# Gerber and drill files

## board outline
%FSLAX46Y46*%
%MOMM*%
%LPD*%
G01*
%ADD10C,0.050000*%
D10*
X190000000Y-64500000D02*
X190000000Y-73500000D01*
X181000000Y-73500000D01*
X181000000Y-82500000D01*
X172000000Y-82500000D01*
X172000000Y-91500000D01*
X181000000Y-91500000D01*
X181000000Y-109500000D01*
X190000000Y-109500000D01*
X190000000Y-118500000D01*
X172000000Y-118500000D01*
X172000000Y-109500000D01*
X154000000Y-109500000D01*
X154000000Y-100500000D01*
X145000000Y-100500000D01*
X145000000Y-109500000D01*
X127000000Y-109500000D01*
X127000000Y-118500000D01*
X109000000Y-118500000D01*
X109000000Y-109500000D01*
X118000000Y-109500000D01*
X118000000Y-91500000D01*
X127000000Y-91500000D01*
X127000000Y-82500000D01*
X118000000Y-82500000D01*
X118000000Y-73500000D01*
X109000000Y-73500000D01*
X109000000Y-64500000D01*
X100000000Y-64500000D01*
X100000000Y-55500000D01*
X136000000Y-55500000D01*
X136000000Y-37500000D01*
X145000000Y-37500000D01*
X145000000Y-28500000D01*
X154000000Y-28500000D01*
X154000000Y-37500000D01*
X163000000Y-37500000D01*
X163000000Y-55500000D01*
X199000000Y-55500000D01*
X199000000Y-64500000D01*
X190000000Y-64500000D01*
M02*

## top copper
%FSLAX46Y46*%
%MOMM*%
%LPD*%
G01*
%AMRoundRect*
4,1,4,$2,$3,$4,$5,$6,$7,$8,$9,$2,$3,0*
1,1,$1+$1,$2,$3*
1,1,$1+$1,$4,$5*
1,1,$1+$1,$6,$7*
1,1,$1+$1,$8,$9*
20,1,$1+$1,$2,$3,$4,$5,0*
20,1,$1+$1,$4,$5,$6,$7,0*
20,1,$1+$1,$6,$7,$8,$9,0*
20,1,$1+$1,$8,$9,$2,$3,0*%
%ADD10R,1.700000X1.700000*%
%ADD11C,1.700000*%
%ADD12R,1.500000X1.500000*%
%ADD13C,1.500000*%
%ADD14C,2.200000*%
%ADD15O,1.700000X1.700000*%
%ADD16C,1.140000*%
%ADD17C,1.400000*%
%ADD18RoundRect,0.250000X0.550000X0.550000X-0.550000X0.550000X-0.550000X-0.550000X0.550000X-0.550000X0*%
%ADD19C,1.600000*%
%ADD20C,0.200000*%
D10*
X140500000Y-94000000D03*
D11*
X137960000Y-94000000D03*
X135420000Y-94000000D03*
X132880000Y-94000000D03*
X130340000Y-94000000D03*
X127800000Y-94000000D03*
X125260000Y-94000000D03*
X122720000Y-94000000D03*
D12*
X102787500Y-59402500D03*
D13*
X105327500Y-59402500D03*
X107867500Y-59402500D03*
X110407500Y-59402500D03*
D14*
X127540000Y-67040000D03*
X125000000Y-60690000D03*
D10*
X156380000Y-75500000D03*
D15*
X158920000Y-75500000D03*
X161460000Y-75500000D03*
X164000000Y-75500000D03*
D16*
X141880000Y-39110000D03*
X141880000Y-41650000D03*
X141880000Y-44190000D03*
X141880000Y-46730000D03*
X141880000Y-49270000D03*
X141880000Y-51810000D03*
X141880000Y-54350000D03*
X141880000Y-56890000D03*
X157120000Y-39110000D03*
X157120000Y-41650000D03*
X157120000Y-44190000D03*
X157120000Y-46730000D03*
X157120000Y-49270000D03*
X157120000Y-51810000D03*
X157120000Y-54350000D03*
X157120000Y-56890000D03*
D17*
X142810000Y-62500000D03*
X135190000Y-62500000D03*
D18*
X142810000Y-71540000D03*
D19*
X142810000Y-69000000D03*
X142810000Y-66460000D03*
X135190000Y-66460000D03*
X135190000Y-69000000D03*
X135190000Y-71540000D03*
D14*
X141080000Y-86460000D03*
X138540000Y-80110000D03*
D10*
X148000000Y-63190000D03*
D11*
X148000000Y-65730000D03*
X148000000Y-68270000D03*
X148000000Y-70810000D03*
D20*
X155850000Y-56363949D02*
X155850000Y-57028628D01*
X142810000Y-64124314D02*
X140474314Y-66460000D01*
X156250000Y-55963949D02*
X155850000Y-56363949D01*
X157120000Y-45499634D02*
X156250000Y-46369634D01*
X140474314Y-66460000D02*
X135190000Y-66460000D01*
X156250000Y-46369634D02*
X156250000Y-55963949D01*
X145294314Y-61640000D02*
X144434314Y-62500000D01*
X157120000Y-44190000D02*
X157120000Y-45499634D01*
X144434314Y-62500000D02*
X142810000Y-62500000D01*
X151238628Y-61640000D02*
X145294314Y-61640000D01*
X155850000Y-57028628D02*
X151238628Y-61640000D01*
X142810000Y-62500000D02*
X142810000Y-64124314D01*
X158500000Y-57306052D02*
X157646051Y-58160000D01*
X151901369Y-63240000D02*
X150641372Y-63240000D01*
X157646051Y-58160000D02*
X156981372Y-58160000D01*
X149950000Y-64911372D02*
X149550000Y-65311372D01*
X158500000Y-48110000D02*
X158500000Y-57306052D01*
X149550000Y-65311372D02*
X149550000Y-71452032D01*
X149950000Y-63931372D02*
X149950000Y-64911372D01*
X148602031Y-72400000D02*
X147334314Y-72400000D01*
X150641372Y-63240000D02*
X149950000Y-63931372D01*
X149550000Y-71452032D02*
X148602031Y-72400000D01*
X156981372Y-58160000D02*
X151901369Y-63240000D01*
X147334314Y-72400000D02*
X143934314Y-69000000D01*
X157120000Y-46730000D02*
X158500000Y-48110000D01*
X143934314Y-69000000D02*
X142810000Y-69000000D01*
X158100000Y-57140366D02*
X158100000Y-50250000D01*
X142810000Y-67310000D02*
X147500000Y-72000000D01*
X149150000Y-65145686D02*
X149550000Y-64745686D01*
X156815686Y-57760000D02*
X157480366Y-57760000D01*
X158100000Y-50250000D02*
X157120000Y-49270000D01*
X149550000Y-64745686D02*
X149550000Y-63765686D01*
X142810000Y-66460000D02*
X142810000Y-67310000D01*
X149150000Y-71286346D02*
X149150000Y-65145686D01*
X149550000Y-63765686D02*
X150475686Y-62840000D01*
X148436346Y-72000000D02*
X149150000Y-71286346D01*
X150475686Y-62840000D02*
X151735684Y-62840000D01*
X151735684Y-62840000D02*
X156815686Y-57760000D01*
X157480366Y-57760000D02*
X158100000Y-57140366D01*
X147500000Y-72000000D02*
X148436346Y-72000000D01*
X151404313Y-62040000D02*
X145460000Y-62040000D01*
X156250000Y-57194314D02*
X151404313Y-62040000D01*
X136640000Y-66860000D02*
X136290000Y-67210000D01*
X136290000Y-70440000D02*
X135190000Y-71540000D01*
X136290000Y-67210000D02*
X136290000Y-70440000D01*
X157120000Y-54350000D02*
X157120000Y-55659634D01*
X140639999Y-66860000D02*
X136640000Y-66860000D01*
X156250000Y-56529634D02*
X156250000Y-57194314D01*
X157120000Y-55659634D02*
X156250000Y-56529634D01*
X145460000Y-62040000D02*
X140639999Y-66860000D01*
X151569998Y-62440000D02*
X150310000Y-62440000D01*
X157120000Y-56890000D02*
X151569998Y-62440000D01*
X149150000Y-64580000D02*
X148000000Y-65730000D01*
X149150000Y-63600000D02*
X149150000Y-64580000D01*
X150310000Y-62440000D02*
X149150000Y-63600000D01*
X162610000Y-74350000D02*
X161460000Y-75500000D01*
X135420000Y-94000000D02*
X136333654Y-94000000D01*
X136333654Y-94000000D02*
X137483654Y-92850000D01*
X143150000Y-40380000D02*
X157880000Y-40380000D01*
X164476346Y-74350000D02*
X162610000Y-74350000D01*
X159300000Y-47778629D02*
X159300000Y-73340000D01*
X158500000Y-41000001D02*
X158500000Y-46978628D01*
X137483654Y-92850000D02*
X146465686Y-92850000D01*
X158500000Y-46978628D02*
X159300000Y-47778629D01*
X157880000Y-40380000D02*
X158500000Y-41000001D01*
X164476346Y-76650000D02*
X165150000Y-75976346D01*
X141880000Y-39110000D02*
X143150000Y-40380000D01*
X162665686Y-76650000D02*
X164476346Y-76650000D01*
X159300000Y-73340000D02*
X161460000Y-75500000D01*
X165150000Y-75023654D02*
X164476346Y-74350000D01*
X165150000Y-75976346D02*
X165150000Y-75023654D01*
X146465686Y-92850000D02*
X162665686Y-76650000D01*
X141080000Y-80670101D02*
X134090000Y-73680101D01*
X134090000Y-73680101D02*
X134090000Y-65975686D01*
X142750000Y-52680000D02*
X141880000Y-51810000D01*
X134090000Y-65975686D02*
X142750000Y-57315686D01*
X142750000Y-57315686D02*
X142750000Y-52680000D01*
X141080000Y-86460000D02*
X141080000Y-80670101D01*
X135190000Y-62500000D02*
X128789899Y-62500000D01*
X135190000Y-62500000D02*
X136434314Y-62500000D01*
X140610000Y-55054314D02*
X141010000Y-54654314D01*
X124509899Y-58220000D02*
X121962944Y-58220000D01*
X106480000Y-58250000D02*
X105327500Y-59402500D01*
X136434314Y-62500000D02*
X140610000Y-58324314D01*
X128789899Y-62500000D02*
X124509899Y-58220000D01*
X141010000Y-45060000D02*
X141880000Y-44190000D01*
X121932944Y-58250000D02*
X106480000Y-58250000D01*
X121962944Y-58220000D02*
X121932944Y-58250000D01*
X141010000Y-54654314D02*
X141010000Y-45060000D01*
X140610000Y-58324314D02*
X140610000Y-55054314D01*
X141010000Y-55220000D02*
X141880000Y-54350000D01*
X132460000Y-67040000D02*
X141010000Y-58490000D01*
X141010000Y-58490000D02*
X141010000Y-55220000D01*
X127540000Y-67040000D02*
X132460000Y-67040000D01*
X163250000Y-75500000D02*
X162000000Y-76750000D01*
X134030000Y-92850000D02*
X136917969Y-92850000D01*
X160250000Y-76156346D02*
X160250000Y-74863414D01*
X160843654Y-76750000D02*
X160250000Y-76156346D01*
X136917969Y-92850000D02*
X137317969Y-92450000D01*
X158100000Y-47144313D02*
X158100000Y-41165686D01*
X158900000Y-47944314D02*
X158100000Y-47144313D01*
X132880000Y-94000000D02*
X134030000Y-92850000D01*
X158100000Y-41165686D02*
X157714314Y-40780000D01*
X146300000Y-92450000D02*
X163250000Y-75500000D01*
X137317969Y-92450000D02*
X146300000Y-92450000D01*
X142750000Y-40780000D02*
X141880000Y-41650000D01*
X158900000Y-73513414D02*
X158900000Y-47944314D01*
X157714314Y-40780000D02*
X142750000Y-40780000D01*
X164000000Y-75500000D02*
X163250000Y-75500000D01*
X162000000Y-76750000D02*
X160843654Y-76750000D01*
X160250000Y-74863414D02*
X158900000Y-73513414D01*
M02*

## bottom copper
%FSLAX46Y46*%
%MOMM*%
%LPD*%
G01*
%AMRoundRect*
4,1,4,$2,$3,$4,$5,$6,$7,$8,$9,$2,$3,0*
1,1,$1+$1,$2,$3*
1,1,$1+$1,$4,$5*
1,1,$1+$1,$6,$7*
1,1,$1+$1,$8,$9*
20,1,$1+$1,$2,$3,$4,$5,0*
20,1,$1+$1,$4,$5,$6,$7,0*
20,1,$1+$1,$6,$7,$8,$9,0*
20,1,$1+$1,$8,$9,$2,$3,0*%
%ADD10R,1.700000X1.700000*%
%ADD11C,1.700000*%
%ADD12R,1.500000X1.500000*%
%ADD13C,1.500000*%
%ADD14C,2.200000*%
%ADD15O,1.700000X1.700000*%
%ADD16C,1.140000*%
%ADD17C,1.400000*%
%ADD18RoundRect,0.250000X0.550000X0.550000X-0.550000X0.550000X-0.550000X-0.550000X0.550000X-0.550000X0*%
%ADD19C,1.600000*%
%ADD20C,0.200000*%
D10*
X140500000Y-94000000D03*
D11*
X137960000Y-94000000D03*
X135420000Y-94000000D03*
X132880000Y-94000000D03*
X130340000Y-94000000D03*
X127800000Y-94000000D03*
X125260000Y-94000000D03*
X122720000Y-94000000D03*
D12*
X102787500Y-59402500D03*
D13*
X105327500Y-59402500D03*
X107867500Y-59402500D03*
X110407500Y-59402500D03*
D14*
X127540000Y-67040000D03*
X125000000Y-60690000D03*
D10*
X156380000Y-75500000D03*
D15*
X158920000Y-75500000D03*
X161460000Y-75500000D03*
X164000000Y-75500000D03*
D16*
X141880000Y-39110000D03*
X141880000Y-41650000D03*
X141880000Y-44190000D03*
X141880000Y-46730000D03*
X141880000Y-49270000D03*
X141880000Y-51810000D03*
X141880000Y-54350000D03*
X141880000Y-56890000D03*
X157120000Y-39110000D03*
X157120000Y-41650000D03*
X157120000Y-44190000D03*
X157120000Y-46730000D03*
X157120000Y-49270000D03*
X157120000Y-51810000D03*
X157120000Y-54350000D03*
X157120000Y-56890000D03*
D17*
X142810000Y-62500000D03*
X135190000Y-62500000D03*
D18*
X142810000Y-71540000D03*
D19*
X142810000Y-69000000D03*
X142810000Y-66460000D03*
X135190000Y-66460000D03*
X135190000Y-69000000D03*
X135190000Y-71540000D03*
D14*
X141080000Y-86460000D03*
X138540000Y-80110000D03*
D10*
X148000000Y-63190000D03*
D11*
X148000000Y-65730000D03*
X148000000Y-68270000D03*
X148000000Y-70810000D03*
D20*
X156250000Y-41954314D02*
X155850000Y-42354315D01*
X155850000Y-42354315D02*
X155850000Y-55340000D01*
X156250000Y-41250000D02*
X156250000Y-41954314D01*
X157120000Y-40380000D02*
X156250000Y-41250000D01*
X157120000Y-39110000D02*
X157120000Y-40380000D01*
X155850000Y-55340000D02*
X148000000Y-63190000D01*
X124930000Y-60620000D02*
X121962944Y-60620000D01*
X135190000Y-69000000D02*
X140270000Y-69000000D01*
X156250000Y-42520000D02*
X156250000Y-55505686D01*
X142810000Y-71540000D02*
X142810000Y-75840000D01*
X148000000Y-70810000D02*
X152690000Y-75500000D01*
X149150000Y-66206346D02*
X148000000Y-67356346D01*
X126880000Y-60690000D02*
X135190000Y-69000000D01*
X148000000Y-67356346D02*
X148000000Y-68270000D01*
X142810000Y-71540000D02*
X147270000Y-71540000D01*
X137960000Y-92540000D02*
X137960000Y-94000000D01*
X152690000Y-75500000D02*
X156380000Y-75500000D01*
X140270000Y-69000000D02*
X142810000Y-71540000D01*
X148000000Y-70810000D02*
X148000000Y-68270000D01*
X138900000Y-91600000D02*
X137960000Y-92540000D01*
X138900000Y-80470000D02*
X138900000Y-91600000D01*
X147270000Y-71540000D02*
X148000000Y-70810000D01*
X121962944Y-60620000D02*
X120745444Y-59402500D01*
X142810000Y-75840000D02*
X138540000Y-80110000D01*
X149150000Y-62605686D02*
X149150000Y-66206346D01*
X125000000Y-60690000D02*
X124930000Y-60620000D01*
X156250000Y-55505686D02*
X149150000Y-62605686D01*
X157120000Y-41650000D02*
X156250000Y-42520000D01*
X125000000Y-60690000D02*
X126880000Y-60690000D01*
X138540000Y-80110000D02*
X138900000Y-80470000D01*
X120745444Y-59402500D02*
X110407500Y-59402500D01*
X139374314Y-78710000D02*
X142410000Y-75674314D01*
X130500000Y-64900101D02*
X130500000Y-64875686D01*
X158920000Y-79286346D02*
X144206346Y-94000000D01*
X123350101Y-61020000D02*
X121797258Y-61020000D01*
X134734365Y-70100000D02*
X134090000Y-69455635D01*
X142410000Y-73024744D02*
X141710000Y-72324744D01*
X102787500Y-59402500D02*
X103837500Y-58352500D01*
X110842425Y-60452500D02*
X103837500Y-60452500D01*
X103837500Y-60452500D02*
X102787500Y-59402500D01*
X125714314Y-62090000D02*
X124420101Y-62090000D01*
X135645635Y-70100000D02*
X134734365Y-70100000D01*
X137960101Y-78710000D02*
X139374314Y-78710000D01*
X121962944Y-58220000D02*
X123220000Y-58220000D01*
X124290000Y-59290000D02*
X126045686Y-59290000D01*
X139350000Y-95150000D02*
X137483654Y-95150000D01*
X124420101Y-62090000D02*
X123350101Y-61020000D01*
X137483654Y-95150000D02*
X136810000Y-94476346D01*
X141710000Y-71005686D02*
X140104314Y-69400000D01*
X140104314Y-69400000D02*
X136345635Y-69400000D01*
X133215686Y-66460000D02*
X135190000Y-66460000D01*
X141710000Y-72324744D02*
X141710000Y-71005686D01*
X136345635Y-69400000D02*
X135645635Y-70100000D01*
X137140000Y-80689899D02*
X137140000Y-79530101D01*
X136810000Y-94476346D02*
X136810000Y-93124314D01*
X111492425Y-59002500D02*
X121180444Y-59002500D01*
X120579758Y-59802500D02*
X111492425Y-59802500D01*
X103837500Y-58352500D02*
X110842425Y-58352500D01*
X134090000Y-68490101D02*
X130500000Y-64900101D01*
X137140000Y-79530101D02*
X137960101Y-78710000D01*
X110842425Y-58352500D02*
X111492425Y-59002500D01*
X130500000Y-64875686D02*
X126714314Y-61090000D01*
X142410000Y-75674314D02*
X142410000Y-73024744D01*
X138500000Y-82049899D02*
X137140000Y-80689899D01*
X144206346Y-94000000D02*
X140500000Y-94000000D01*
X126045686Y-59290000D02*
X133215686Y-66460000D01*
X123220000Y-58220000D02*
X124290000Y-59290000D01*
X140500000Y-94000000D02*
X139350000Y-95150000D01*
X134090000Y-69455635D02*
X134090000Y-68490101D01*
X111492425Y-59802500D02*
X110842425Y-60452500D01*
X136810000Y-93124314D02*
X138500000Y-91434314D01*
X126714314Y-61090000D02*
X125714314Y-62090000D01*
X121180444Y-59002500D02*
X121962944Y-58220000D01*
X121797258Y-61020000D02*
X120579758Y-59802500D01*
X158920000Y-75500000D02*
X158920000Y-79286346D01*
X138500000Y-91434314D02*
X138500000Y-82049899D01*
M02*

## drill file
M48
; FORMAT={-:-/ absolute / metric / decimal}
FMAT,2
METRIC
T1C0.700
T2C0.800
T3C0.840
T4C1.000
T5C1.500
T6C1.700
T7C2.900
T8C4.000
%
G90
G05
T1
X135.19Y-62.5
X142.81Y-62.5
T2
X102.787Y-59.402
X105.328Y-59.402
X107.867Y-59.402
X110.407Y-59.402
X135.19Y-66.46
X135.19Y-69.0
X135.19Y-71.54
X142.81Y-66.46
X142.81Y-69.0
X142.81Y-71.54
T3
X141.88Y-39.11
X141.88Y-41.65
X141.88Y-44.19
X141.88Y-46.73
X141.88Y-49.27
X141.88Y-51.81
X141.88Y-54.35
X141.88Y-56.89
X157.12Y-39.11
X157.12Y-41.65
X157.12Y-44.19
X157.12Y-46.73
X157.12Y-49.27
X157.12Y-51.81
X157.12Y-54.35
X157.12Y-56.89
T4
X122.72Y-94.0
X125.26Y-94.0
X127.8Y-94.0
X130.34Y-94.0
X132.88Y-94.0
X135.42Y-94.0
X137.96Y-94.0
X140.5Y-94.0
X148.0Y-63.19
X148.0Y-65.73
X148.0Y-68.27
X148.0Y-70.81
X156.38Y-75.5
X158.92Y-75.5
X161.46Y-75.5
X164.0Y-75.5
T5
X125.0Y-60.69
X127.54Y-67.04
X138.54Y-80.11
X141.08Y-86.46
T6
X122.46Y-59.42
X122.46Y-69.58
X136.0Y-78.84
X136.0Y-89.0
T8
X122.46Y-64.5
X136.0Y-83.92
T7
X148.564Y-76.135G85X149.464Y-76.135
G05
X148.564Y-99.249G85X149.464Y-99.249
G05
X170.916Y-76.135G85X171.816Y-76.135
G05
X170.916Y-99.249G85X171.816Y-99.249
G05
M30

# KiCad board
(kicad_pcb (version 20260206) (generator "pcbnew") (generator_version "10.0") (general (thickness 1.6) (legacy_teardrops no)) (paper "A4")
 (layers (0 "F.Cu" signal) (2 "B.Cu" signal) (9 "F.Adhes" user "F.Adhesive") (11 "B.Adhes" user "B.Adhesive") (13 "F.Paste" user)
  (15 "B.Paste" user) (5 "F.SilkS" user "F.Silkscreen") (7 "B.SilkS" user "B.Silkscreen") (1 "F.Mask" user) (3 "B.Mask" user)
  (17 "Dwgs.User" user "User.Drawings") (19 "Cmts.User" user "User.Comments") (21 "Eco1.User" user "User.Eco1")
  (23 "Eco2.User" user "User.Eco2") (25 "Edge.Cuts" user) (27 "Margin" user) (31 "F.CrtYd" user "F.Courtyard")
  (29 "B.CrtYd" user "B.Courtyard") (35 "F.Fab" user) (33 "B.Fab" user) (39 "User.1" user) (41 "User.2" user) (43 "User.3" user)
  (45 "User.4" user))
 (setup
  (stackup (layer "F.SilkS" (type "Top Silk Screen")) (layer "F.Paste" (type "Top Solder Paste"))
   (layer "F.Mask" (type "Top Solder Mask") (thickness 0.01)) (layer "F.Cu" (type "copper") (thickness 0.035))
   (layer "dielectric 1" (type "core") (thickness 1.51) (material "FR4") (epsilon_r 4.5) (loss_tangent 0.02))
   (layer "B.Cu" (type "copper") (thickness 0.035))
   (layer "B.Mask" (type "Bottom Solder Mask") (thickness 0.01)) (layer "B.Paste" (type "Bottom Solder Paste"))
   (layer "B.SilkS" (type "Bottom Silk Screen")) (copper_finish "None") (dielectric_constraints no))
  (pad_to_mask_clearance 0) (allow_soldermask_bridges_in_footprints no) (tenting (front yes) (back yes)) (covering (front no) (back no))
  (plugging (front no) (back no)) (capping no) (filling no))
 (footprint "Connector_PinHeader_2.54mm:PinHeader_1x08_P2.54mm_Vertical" (layer "F.Cu") (at 140.5 94 -90)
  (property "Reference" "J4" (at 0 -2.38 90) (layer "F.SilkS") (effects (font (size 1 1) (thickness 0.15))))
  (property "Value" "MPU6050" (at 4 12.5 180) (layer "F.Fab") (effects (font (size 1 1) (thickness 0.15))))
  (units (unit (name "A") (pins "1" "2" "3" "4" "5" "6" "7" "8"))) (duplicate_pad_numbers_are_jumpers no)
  (pad "1" thru_hole rect (at 0 0 270) (size 1.7 1.7) (drill 1) (layers "*.Cu" "*.Mask") (remove_unused_layers no) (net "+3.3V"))
  (pad "2" thru_hole circle (at 0 2.54 270) (size 1.7 1.7) (drill 1) (layers "*.Cu" "*.Mask") (remove_unused_layers no) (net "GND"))
  (pad "3" thru_hole circle (at 0 5.08 270) (size 1.7 1.7) (drill 1) (layers "*.Cu" "*.Mask") (remove_unused_layers no) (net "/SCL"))
  (pad "4" thru_hole circle (at 0 7.62 270) (size 1.7 1.7) (drill 1) (layers "*.Cu" "*.Mask") (remove_unused_layers no) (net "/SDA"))
  (pad "5" thru_hole circle (at 0 10.16 270) (size 1.7 1.7) (drill 1) (layers "*.Cu" "*.Mask") (remove_unused_layers no)
   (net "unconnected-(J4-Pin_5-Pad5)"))
  (pad "6" thru_hole circle (at 0 12.7 270) (size 1.7 1.7) (drill 1) (layers "*.Cu" "*.Mask") (remove_unused_layers no)
   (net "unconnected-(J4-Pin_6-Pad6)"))
  (pad "7" thru_hole circle (at 0 15.24 270) (size 1.7 1.7) (drill 1) (layers "*.Cu" "*.Mask") (remove_unused_layers no)
   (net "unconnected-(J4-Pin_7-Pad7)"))
  (pad "8" thru_hole circle (at 0 17.78 270) (size 1.7 1.7) (drill 1) (layers "*.Cu" "*.Mask") (remove_unused_layers no)
   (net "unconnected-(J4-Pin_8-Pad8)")))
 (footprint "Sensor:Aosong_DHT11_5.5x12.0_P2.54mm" (layer "F.Cu") (at 102.7875 59.4025 90)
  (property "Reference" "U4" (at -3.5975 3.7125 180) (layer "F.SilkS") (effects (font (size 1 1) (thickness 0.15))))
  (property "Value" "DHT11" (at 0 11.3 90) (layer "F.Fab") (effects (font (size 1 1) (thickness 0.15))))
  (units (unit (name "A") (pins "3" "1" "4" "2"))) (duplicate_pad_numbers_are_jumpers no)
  (pad "1" thru_hole rect (at 0 0 90) (size 1.5 1.5) (drill 0.8) (layers "*.Cu" "*.Mask") (remove_unused_layers no) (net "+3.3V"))
  (pad "2" thru_hole circle (at 0 2.54 90) (size 1.5 1.5) (drill 0.8) (layers "*.Cu" "*.Mask") (remove_unused_layers no) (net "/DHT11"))
  (pad "3" thru_hole circle (at 0 5.08 90) (size 1.5 1.5) (drill 0.8) (layers "*.Cu" "*.Mask") (remove_unused_layers no)
   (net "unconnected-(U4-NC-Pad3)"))
  (pad "4" thru_hole circle (at 0 7.62 90) (size 1.5 1.5) (drill 0.8) (layers "*.Cu" "*.Mask") (remove_unused_layers no) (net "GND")))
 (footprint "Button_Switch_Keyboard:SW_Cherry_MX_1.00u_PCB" (layer "F.Cu") (at 127.54 67.04 -90)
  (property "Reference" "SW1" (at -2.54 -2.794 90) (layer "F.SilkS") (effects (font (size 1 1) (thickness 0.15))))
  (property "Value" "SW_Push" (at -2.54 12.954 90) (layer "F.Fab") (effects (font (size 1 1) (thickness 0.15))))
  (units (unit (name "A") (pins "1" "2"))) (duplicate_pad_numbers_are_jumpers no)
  (pad "" np_thru_hole circle (at -7.62 5.08 270) (size 1.7 1.7) (drill 1.7) (layers "*.Cu" "*.Mask"))
  (pad "" np_thru_hole circle (at -2.54 5.08 270) (size 4 4) (drill 4) (layers "*.Cu" "*.Mask"))
  (pad "" np_thru_hole circle (at 2.54 5.08 270) (size 1.7 1.7) (drill 1.7) (layers "*.Cu" "*.Mask"))
  (pad "1" thru_hole circle (at 0 0 270) (size 2.2 2.2) (drill 1.5) (layers "*.Cu" "*.Mask") (remove_unused_layers no) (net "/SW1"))
  (pad "2" thru_hole circle (at -6.35 2.54 270) (size 2.2 2.2) (drill 1.5) (layers "*.Cu" "*.Mask") (remove_unused_layers no) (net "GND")))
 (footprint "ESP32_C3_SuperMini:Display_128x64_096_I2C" (layer "F.Cu") (at 160.19 75.5)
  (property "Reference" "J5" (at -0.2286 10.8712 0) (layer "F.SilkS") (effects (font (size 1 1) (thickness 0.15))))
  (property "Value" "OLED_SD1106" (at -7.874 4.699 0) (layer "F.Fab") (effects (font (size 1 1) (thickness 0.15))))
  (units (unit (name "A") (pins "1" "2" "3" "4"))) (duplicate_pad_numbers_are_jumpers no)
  (pad "" np_thru_hole oval (at -11.176 0.635) (size 3.8 2.9) (drill oval 3.8 2.9) (layers "*.Cu" "*.Mask"))
  (pad "" np_thru_hole oval (at -11.176 23.749) (size 3.8 2.9) (drill oval 3.8 2.9) (layers "*.Cu" "*.Mask"))
  (pad "" np_thru_hole oval (at 11.176 0.635) (size 3.8 2.9) (drill oval 3.8 2.9) (layers "*.Cu" "*.Mask"))
  (pad "" np_thru_hole oval (at 11.176 23.749) (size 3.8 2.9) (drill oval 3.8 2.9) (layers "*.Cu" "*.Mask"))
  (pad "1" thru_hole rect (at -3.81 0 90) (size 1.7 1.7) (drill 1) (layers "*.Cu" "*.Mask") (remove_unused_layers no) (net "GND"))
  (pad "2" thru_hole oval (at -1.27 0 90) (size 1.7 1.7) (drill 1) (layers "*.Cu" "*.Mask") (remove_unused_layers no) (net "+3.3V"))
  (pad "3" thru_hole oval (at 1.27 0 90) (size 1.7 1.7) (drill 1) (layers "*.Cu" "*.Mask") (remove_unused_layers no) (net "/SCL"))
  (pad "4" thru_hole oval (at 3.81 0 90) (size 1.7 1.7) (drill 1) (layers "*.Cu" "*.Mask") (remove_unused_layers no) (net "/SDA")))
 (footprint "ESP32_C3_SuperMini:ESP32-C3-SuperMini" (layer "F.Cu") (at 149.5 48)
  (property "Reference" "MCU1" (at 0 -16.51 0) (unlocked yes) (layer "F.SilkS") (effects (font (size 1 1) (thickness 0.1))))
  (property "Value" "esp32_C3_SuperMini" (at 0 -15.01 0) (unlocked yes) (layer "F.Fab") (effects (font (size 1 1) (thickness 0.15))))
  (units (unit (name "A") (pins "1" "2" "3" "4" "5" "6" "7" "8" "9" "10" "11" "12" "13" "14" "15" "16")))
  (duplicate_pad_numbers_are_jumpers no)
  (pad "1" thru_hole circle (at -7.62 -8.89) (size 1.14 1.14) (drill 0.84) (layers "*.Cu" "*.Mask") (remove_unused_layers no) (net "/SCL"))
  (pad "2" thru_hole circle (at -7.62 -6.35) (size 1.14 1.14) (drill 0.84) (layers "*.Cu" "*.Mask") (remove_unused_layers no) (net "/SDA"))
  (pad "3" thru_hole circle (at -7.62 -3.81) (size 1.14 1.14) (drill 0.84) (layers "*.Cu" "*.Mask") (remove_unused_layers no) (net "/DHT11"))
  (pad "4" thru_hole circle (at -7.62 -1.27) (size 1.14 1.14) (drill 0.84) (layers "*.Cu" "*.Mask") (remove_unused_layers no)
   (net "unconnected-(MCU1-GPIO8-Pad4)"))
  (pad "5" thru_hole circle (at -7.62 1.27) (size 1.14 1.14) (drill 0.84) (layers "*.Cu" "*.Mask") (remove_unused_layers no)
   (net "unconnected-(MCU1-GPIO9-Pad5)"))
  (pad "6" thru_hole circle (at -7.62 3.81) (size 1.14 1.14) (drill 0.84) (layers "*.Cu" "*.Mask") (remove_unused_layers no) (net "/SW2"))
  (pad "7" thru_hole circle (at -7.62 6.35) (size 1.14 1.14) (drill 0.84) (layers "*.Cu" "*.Mask") (remove_unused_layers no) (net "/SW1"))
  (pad "8" thru_hole circle (at -7.62 8.89) (size 1.14 1.14) (drill 0.84) (layers "*.Cu" "*.Mask") (remove_unused_layers no)
   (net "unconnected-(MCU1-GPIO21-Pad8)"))
  (pad "9" thru_hole circle (at 7.62 -8.89) (size 1.14 1.14) (drill 0.84) (layers "*.Cu" "*.Mask") (remove_unused_layers no) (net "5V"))
  (pad "10" thru_hole circle (at 7.62 -6.35) (size 1.14 1.14) (drill 0.84) (layers "*.Cu" "*.Mask") (remove_unused_layers no) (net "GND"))
  (pad "11" thru_hole circle (at 7.62 -3.81) (size 1.14 1.14) (drill 0.84) (layers "*.Cu" "*.Mask") (remove_unused_layers no) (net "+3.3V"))
  (pad "12" thru_hole circle (at 7.62 -1.27) (size 1.14 1.14) (drill 0.84) (layers "*.Cu" "*.Mask") (remove_unused_layers no) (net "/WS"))
  (pad "13" thru_hole circle (at 7.62 1.27) (size 1.14 1.14) (drill 0.84) (layers "*.Cu" "*.Mask") (remove_unused_layers no) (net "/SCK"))
  (pad "14" thru_hole circle (at 7.62 3.81) (size 1.14 1.14) (drill 0.84) (layers "*.Cu" "*.Mask") (remove_unused_layers no)
   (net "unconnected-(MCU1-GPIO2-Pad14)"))
  (pad "15" thru_hole circle (at 7.62 6.35) (size 1.14 1.14) (drill 0.84) (layers "*.Cu" "*.Mask") (remove_unused_layers no) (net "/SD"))
  (pad "16" thru_hole circle (at 7.62 8.89) (size 1.14 1.14) (drill 0.84) (layers "*.Cu" "*.Mask") (remove_unused_layers no) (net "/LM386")))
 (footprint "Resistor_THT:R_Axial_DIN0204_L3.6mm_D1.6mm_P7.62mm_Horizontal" (layer "F.Cu") (at 142.81 62.5 180)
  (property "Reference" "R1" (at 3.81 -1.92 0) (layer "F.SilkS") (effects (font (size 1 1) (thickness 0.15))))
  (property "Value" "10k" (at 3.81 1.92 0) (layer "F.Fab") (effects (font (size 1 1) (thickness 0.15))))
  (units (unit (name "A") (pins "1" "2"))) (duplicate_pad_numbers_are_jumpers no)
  (pad "1" thru_hole circle (at 0 0 180) (size 1.4 1.4) (drill 0.7) (layers "*.Cu" "*.Mask") (remove_unused_layers no) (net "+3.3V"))
  (pad "2" thru_hole circle (at 7.62 0 180) (size 1.4 1.4) (drill 0.7) (layers "*.Cu" "*.Mask") (remove_unused_layers no) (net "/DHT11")))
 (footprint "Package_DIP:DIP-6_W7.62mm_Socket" (layer "F.Cu") (at 142.81 71.54 180)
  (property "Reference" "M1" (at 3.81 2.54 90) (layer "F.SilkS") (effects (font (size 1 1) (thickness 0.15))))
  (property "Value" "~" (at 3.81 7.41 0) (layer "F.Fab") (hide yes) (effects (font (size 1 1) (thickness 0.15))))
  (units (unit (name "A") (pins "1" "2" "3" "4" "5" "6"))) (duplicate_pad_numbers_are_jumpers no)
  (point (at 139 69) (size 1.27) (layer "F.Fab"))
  (pad "1" thru_hole roundrect (at 0 0 180) (size 1.6 1.6) (drill 0.8) (layers "*.Cu" "*.Mask") (remove_unused_layers no)
   (roundrect_rratio 0.15625) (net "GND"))
  (pad "2" thru_hole circle (at 0 2.54 180) (size 1.6 1.6) (drill 0.8) (layers "*.Cu" "*.Mask") (remove_unused_layers no) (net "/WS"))
  (pad "3" thru_hole circle (at 0 5.08 180) (size 1.6 1.6) (drill 0.8) (layers "*.Cu" "*.Mask") (remove_unused_layers no) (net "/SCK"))
  (pad "4" thru_hole circle (at 7.62 5.08 180) (size 1.6 1.6) (drill 0.8) (layers "*.Cu" "*.Mask") (remove_unused_layers no) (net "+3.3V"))
  (pad "5" thru_hole circle (at 7.62 2.54 180) (size 1.6 1.6) (drill 0.8) (layers "*.Cu" "*.Mask") (remove_unused_layers no) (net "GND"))
  (pad "6" thru_hole circle (at 7.62 0 180) (size 1.6 1.6) (drill 0.8) (layers "*.Cu" "*.Mask") (remove_unused_layers no) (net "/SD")))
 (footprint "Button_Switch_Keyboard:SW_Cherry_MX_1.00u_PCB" (layer "F.Cu") (at 141.08 86.46 -90)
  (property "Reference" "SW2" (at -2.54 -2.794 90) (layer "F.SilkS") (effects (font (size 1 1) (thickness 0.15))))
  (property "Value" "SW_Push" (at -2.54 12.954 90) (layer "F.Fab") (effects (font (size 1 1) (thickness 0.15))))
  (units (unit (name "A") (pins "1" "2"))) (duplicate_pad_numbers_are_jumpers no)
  (pad "" np_thru_hole circle (at -7.62 5.08 270) (size 1.7 1.7) (drill 1.7) (layers "*.Cu" "*.Mask"))
  (pad "" np_thru_hole circle (at -2.54 5.08 270) (size 4 4) (drill 4) (layers "*.Cu" "*.Mask"))
  (pad "" np_thru_hole circle (at 2.54 5.08 270) (size 1.7 1.7) (drill 1.7) (layers "*.Cu" "*.Mask"))
  (pad "1" thru_hole circle (at 0 0 270) (size 2.2 2.2) (drill 1.5) (layers "*.Cu" "*.Mask") (remove_unused_layers no) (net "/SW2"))
  (pad "2" thru_hole circle (at -6.35 2.54 270) (size 2.2 2.2) (drill 1.5) (layers "*.Cu" "*.Mask") (remove_unused_layers no) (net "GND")))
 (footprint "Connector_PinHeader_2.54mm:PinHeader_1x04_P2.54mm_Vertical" (layer "F.Cu") (at 148 63.19)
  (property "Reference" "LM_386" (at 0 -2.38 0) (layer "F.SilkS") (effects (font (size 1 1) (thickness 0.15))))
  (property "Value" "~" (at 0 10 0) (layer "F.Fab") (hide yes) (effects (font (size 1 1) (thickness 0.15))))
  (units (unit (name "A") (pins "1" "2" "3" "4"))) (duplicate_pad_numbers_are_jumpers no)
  (pad "1" thru_hole rect (at 0 0) (size 1.7 1.7) (drill 1) (layers "*.Cu" "*.Mask") (remove_unused_layers no) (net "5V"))
  (pad "2" thru_hole circle (at 0 2.54) (size 1.7 1.7) (drill 1) (layers "*.Cu" "*.Mask") (remove_unused_layers no) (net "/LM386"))
  (pad "3" thru_hole circle (at 0 5.08) (size 1.7 1.7) (drill 1) (layers "*.Cu" "*.Mask") (remove_unused_layers no) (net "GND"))
  (pad "4" thru_hole circle (at 0 7.62) (size 1.7 1.7) (drill 1) (layers "*.Cu" "*.Mask") (remove_unused_layers no) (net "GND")))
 (gr_poly
  (pts (xy 190 64.5) (xy 190 73.5) (xy 181 73.5) (xy 181 82.5) (xy 172 82.5) (xy 172 91.5) (xy 181 91.5) (xy 181 109.5) (xy 190 109.5)
   (xy 190 118.5) (xy 172 118.5) (xy 172 109.5) (xy 154 109.5) (xy 154 100.5) (xy 145 100.5) (xy 145 109.5) (xy 127 109.5) (xy 127 118.5)
   (xy 109 118.5) (xy 109 109.5) (xy 118 109.5) (xy 118 91.5) (xy 127 91.5) (xy 127 82.5) (xy 118 82.5) (xy 118 73.5) (xy 109 73.5)
   (xy 109 64.5) (xy 100 64.5) (xy 100 55.5) (xy 136 55.5) (xy 136 37.5) (xy 145 37.5) (xy 145 28.5) (xy 154 28.5) (xy 154 37.5)
   (xy 163 37.5) (xy 163 55.5) (xy 199 55.5) (xy 199 64.5))
  (stroke (width 0.05) (type solid)) (fill no) (layer "Edge.Cuts"))
 (segment (start 156.25 41.954314) (end 155.85 42.354315) (width 0.2) (layer "B.Cu") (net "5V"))
 (segment (start 155.85 42.354315) (end 155.85 55.34) (width 0.2) (layer "B.Cu") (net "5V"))
 (segment (start 156.25 41.25) (end 156.25 41.954314) (width 0.2) (layer "B.Cu") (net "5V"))
 (segment (start 157.12 40.38) (end 156.25 41.25) (width 0.2) (layer "B.Cu") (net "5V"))
 (segment (start 157.12 39.11) (end 157.12 40.38) (width 0.2) (layer "B.Cu") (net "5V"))
 (segment (start 155.85 55.34) (end 148 63.19) (width 0.2) (layer "B.Cu") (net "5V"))
 (segment (start 124.93 60.62) (end 121.962944 60.62) (width 0.2) (layer "B.Cu") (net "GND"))
 (segment (start 135.19 69) (end 140.27 69) (width 0.2) (layer "B.Cu") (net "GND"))
 (segment (start 156.25 42.52) (end 156.25 55.505686) (width 0.2) (layer "B.Cu") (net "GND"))
 (segment (start 142.81 71.54) (end 142.81 75.84) (width 0.2) (layer "B.Cu") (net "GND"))
 (segment (start 148 70.81) (end 152.69 75.5) (width 0.2) (layer "B.Cu") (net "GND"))
 (segment (start 149.15 66.206346) (end 148 67.356346) (width 0.2) (layer "B.Cu") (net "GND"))
 (segment (start 126.88 60.69) (end 135.19 69) (width 0.2) (layer "B.Cu") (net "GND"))
 (segment (start 148 67.356346) (end 148 68.27) (width 0.2) (layer "B.Cu") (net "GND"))
 (segment (start 142.81 71.54) (end 147.27 71.54) (width 0.2) (layer "B.Cu") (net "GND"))
 (segment (start 137.96 92.54) (end 137.96 94) (width 0.2) (layer "B.Cu") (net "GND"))
 (segment (start 152.69 75.5) (end 156.38 75.5) (width 0.2) (layer "B.Cu") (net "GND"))
 (segment (start 140.27 69) (end 142.81 71.54) (width 0.2) (layer "B.Cu") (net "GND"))
 (segment (start 148 70.81) (end 148 68.27) (width 0.2) (layer "B.Cu") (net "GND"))
 (segment (start 138.9 91.6) (end 137.96 92.54) (width 0.2) (layer "B.Cu") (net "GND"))
 (segment (start 138.9 80.47) (end 138.9 91.6) (width 0.2) (layer "B.Cu") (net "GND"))
 (segment (start 147.27 71.54) (end 148 70.81) (width 0.2) (layer "B.Cu") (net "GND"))
 (segment (start 121.962944 60.62) (end 120.745444 59.4025) (width 0.2) (layer "B.Cu") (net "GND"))
 (segment (start 142.81 75.84) (end 138.54 80.11) (width 0.2) (layer "B.Cu") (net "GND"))
 (segment (start 149.15 62.605686) (end 149.15 66.206346) (width 0.2) (layer "B.Cu") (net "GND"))
 (segment (start 125 60.69) (end 124.93 60.62) (width 0.2) (layer "B.Cu") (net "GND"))
 (segment (start 156.25 55.505686) (end 149.15 62.605686) (width 0.2) (layer "B.Cu") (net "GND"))
 (segment (start 157.12 41.65) (end 156.25 42.52) (width 0.2) (layer "B.Cu") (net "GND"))
 (segment (start 125 60.69) (end 126.88 60.69) (width 0.2) (layer "B.Cu") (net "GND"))
 (segment (start 138.54 80.11) (end 138.9 80.47) (width 0.2) (layer "B.Cu") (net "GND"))
 (segment (start 120.745444 59.4025) (end 110.4075 59.4025) (width 0.2) (layer "B.Cu") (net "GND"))
 (segment (start 155.85 56.363949) (end 155.85 57.028628) (width 0.2) (layer "F.Cu") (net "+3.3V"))
 (segment (start 142.81 64.124314) (end 140.474314 66.46) (width 0.2) (layer "F.Cu") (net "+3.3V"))
 (segment (start 156.25 55.963949) (end 155.85 56.363949) (width 0.2) (layer "F.Cu") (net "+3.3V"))
 (segment (start 157.12 45.499634) (end 156.25 46.369634) (width 0.2) (layer "F.Cu") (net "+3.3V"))
 (segment (start 140.474314 66.46) (end 135.19 66.46) (width 0.2) (layer "F.Cu") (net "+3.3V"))
 (segment (start 156.25 46.369634) (end 156.25 55.963949) (width 0.2) (layer "F.Cu") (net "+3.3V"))
 (segment (start 145.294314 61.64) (end 144.434314 62.5) (width 0.2) (layer "F.Cu") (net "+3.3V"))
 (segment (start 157.12 44.19) (end 157.12 45.499634) (width 0.2) (layer "F.Cu") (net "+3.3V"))
 (segment (start 144.434314 62.5) (end 142.81 62.5) (width 0.2) (layer "F.Cu") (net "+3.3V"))
 (segment (start 151.238628 61.64) (end 145.294314 61.64) (width 0.2) (layer "F.Cu") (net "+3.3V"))
 (segment (start 155.85 57.028628) (end 151.238628 61.64) (width 0.2) (layer "F.Cu") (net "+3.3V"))
 (segment (start 142.81 62.5) (end 142.81 64.124314) (width 0.2) (layer "F.Cu") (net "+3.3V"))
 (segment (start 139.374314 78.71) (end 142.41 75.674314) (width 0.2) (layer "B.Cu") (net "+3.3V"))
 (segment (start 130.5 64.900101) (end 130.5 64.875686) (width 0.2) (layer "B.Cu") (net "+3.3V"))
 (segment (start 158.92 79.286346) (end 144.206346 94) (width 0.2) (layer "B.Cu") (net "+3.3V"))
 (segment (start 123.350101 61.02) (end 121.797258 61.02) (width 0.2) (layer "B.Cu") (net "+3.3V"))
 (segment (start 134.734365 70.1) (end 134.09 69.455635) (width 0.2) (layer "B.Cu") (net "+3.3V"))
 (segment (start 142.41 73.024744) (end 141.71 72.324744) (width 0.2) (layer "B.Cu") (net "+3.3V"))
 (segment (start 102.7875 59.4025) (end 103.8375 58.3525) (width 0.2) (layer "B.Cu") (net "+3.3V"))
 (segment (start 110.842425 60.4525) (end 103.8375 60.4525) (width 0.2) (layer "B.Cu") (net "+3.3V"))
 (segment (start 103.8375 60.4525) (end 102.7875 59.4025) (width 0.2) (layer "B.Cu") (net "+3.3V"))
 (segment (start 125.714314 62.09) (end 124.420101 62.09) (width 0.2) (layer "B.Cu") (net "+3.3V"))
 (segment (start 135.645635 70.1) (end 134.734365 70.1) (width 0.2) (layer "B.Cu") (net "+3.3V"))
 (segment (start 137.960101 78.71) (end 139.374314 78.71) (width 0.2) (layer "B.Cu") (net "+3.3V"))
 (segment (start 121.962944 58.22) (end 123.22 58.22) (width 0.2) (layer "B.Cu") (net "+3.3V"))
 (segment (start 124.29 59.29) (end 126.045686 59.29) (width 0.2) (layer "B.Cu") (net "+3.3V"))
 (segment (start 139.35 95.15) (end 137.483654 95.15) (width 0.2) (layer "B.Cu") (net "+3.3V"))
 (segment (start 124.420101 62.09) (end 123.350101 61.02) (width 0.2) (layer "B.Cu") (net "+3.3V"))
 (segment (start 137.483654 95.15) (end 136.81 94.476346) (width 0.2) (layer "B.Cu") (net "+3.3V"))
 (segment (start 141.71 71.005686) (end 140.104314 69.4) (width 0.2) (layer "B.Cu") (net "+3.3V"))
 (segment (start 140.104314 69.4) (end 136.345635 69.4) (width 0.2) (layer "B.Cu") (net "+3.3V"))
 (segment (start 133.215686 66.46) (end 135.19 66.46) (width 0.2) (layer "B.Cu") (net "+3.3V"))
 (segment (start 141.71 72.324744) (end 141.71 71.005686) (width 0.2) (layer "B.Cu") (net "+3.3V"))
 (segment (start 136.345635 69.4) (end 135.645635 70.1) (width 0.2) (layer "B.Cu") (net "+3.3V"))
 (segment (start 137.14 80.689899) (end 137.14 79.530101) (width 0.2) (layer "B.Cu") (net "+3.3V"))
 (segment (start 136.81 94.476346) (end 136.81 93.124314) (width 0.2) (layer "B.Cu") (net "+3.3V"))
 (segment (start 111.492425 59.0025) (end 121.180444 59.0025) (width 0.2) (layer "B.Cu") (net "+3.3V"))
 (segment (start 120.579758 59.8025) (end 111.492425 59.8025) (width 0.2) (layer "B.Cu") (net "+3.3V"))
 (segment (start 103.8375 58.3525) (end 110.842425 58.3525) (width 0.2) (layer "B.Cu") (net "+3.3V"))
 (segment (start 134.09 68.490101) (end 130.5 64.900101) (width 0.2) (layer "B.Cu") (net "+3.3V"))
 (segment (start 137.14 79.530101) (end 137.960101 78.71) (width 0.2) (layer "B.Cu") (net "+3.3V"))
 (segment (start 110.842425 58.3525) (end 111.492425 59.0025) (width 0.2) (layer "B.Cu") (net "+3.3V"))
 (segment (start 130.5 64.875686) (end 126.714314 61.09) (width 0.2) (layer "B.Cu") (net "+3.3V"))
 (segment (start 142.41 75.674314) (end 142.41 73.024744) (width 0.2) (layer "B.Cu") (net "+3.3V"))
 (segment (start 138.5 82.049899) (end 137.14 80.689899) (width 0.2) (layer "B.Cu") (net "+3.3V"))
 (segment (start 144.206346 94) (end 140.5 94) (width 0.2) (layer "B.Cu") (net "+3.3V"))
 (segment (start 126.045686 59.29) (end 133.215686 66.46) (width 0.2) (layer "B.Cu") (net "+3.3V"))
 (segment (start 123.22 58.22) (end 124.29 59.29) (width 0.2) (layer "B.Cu") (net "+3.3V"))
 (segment (start 140.5 94) (end 139.35 95.15) (width 0.2) (layer "B.Cu") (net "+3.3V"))
 (segment (start 134.09 69.455635) (end 134.09 68.490101) (width 0.2) (layer "B.Cu") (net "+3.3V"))
 (segment (start 111.492425 59.8025) (end 110.842425 60.4525) (width 0.2) (layer "B.Cu") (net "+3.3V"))
 (segment (start 136.81 93.124314) (end 138.5 91.434314) (width 0.2) (layer "B.Cu") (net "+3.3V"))
 (segment (start 126.714314 61.09) (end 125.714314 62.09) (width 0.2) (layer "B.Cu") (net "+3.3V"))
 (segment (start 121.180444 59.0025) (end 121.962944 58.22) (width 0.2) (layer "B.Cu") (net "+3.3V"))
 (segment (start 121.797258 61.02) (end 120.579758 59.8025) (width 0.2) (layer "B.Cu") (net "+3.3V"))
 (segment (start 158.92 75.5) (end 158.92 79.286346) (width 0.2) (layer "B.Cu") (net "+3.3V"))
 (segment (start 138.5 91.434314) (end 138.5 82.049899) (width 0.2) (layer "B.Cu") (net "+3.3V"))
 (segment (start 158.5 57.306052) (end 157.646051 58.16) (width 0.2) (layer "F.Cu") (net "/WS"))
 (segment (start 151.901369 63.24) (end 150.641372 63.24) (width 0.2) (layer "F.Cu") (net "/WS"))
 (segment (start 157.646051 58.16) (end 156.981372 58.16) (width 0.2) (layer "F.Cu") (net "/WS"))
 (segment (start 149.95 64.911372) (end 149.55 65.311372) (width 0.2) (layer "F.Cu") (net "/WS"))
 (segment (start 158.5 48.11) (end 158.5 57.306052) (width 0.2) (layer "F.Cu") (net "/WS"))
 (segment (start 149.55 65.311372) (end 149.55 71.452032) (width 0.2) (layer "F.Cu") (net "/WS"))
 (segment (start 149.95 63.931372) (end 149.95 64.911372) (width 0.2) (layer "F.Cu") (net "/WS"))
 (segment (start 148.602031 72.4) (end 147.334314 72.4) (width 0.2) (layer "F.Cu") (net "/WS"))
 (segment (start 150.641372 63.24) (end 149.95 63.931372) (width 0.2) (layer "F.Cu") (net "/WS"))
 (segment (start 149.55 71.452032) (end 148.602031 72.4) (width 0.2) (layer "F.Cu") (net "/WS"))
 (segment (start 156.981372 58.16) (end 151.901369 63.24) (width 0.2) (layer "F.Cu") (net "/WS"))
 (segment (start 147.334314 72.4) (end 143.934314 69) (width 0.2) (layer "F.Cu") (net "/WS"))
 (segment (start 157.12 46.73) (end 158.5 48.11) (width 0.2) (layer "F.Cu") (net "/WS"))
 (segment (start 143.934314 69) (end 142.81 69) (width 0.2) (layer "F.Cu") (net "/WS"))
 (segment (start 158.1 57.140366) (end 158.1 50.25) (width 0.2) (layer "F.Cu") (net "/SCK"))
 (segment (start 142.81 67.31) (end 147.5 72) (width 0.2) (layer "F.Cu") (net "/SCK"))
 (segment (start 149.15 65.145686) (end 149.55 64.745686) (width 0.2) (layer "F.Cu") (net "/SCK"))
 (segment (start 156.815686 57.76) (end 157.480366 57.76) (width 0.2) (layer "F.Cu") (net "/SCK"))
 (segment (start 158.1 50.25) (end 157.12 49.27) (width 0.2) (layer "F.Cu") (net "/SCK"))
 (segment (start 149.55 64.745686) (end 149.55 63.765686) (width 0.2) (layer "F.Cu") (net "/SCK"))
 (segment (start 142.81 66.46) (end 142.81 67.31) (width 0.2) (layer "F.Cu") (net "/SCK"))
 (segment (start 149.15 71.286346) (end 149.15 65.145686) (width 0.2) (layer "F.Cu") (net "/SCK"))
 (segment (start 149.55 63.765686) (end 150.475686 62.84) (width 0.2) (layer "F.Cu") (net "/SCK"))
 (segment (start 148.436346 72) (end 149.15 71.286346) (width 0.2) (layer "F.Cu") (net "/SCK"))
 (segment (start 150.475686 62.84) (end 151.735684 62.84) (width 0.2) (layer "F.Cu") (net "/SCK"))
 (segment (start 151.735684 62.84) (end 156.815686 57.76) (width 0.2) (layer "F.Cu") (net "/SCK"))
 (segment (start 157.480366 57.76) (end 158.1 57.140366) (width 0.2) (layer "F.Cu") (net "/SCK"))
 (segment (start 147.5 72) (end 148.436346 72) (width 0.2) (layer "F.Cu") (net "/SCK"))
 (segment (start 151.404313 62.04) (end 145.46 62.04) (width 0.2) (layer "F.Cu") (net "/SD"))
 (segment (start 156.25 57.194314) (end 151.404313 62.04) (width 0.2) (layer "F.Cu") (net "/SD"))
 (segment (start 136.64 66.86) (end 136.29 67.21) (width 0.2) (layer "F.Cu") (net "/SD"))
 (segment (start 136.29 70.44) (end 135.19 71.54) (width 0.2) (layer "F.Cu") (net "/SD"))
 (segment (start 136.29 67.21) (end 136.29 70.44) (width 0.2) (layer "F.Cu") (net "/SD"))
 (segment (start 157.12 54.35) (end 157.12 55.659634) (width 0.2) (layer "F.Cu") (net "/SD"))
 (segment (start 140.639999 66.86) (end 136.64 66.86) (width 0.2) (layer "F.Cu") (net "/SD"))
 (segment (start 156.25 56.529634) (end 156.25 57.194314) (width 0.2) (layer "F.Cu") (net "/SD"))
 (segment (start 157.12 55.659634) (end 156.25 56.529634) (width 0.2) (layer "F.Cu") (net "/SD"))
 (segment (start 145.46 62.04) (end 140.639999 66.86) (width 0.2) (layer "F.Cu") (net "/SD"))
 (segment (start 151.569998 62.44) (end 150.31 62.44) (width 0.2) (layer "F.Cu") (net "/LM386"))
 (segment (start 157.12 56.89) (end 151.569998 62.44) (width 0.2) (layer "F.Cu") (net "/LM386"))
 (segment (start 149.15 64.58) (end 148 65.73) (width 0.2) (layer "F.Cu") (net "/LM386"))
 (segment (start 149.15 63.6) (end 149.15 64.58) (width 0.2) (layer "F.Cu") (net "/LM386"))
 (segment (start 150.31 62.44) (end 149.15 63.6) (width 0.2) (layer "F.Cu") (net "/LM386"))
 (segment (start 162.61 74.35) (end 161.46 75.5) (width 0.2) (layer "F.Cu") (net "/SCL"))
 (segment (start 135.42 94) (end 136.333654 94) (width 0.2) (layer "F.Cu") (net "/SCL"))
 (segment (start 136.333654 94) (end 137.483654 92.85) (width 0.2) (layer "F.Cu") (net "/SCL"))
 (segment (start 143.15 40.38) (end 157.88 40.38) (width 0.2) (layer "F.Cu") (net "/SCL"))
 (segment (start 164.476346 74.35) (end 162.61 74.35) (width 0.2) (layer "F.Cu") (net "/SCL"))
 (segment (start 159.3 47.778629) (end 159.3 73.34) (width 0.2) (layer "F.Cu") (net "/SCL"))
 (segment (start 158.5 41.000001) (end 158.5 46.978628) (width 0.2) (layer "F.Cu") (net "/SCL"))
 (segment (start 137.483654 92.85) (end 146.465686 92.85) (width 0.2) (layer "F.Cu") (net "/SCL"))
 (segment (start 158.5 46.978628) (end 159.3 47.778629) (width 0.2) (layer "F.Cu") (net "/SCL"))
 (segment (start 157.88 40.38) (end 158.5 41.000001) (width 0.2) (layer "F.Cu") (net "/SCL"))
 (segment (start 164.476346 76.65) (end 165.15 75.976346) (width 0.2) (layer "F.Cu") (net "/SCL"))
 (segment (start 141.88 39.11) (end 143.15 40.38) (width 0.2) (layer "F.Cu") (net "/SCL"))
 (segment (start 162.665686 76.65) (end 164.476346 76.65) (width 0.2) (layer "F.Cu") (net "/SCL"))
 (segment (start 159.3 73.34) (end 161.46 75.5) (width 0.2) (layer "F.Cu") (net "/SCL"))
 (segment (start 165.15 75.023654) (end 164.476346 74.35) (width 0.2) (layer "F.Cu") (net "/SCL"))
 (segment (start 165.15 75.976346) (end 165.15 75.023654) (width 0.2) (layer "F.Cu") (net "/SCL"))
 (segment (start 146.465686 92.85) (end 162.665686 76.65) (width 0.2) (layer "F.Cu") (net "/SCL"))
 (segment (start 141.08 80.670101) (end 134.09 73.680101) (width 0.2) (layer "F.Cu") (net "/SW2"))
 (segment (start 134.09 73.680101) (end 134.09 65.975686) (width 0.2) (layer "F.Cu") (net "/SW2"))
 (segment (start 142.75 52.68) (end 141.88 51.81) (width 0.2) (layer "F.Cu") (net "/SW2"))
 (segment (start 134.09 65.975686) (end 142.75 57.315686) (width 0.2) (layer "F.Cu") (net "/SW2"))
 (segment (start 142.75 57.315686) (end 142.75 52.68) (width 0.2) (layer "F.Cu") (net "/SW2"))
 (segment (start 141.08 86.46) (end 141.08 80.670101) (width 0.2) (layer "F.Cu") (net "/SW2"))
 (segment (start 135.19 62.5) (end 128.789899 62.5) (width 0.2) (layer "F.Cu") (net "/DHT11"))
 (segment (start 135.19 62.5) (end 136.434314 62.5) (width 0.2) (layer "F.Cu") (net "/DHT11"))
 (segment (start 140.61 55.054314) (end 141.01 54.654314) (width 0.2) (layer "F.Cu") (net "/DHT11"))
 (segment (start 124.509899 58.22) (end 121.962944 58.22) (width 0.2) (layer "F.Cu") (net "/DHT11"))
 (segment (start 106.48 58.25) (end 105.3275 59.4025) (width 0.2) (layer "F.Cu") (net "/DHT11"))
 (segment (start 136.434314 62.5) (end 140.61 58.324314) (width 0.2) (layer "F.Cu") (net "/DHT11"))
 (segment (start 128.789899 62.5) (end 124.509899 58.22) (width 0.2) (layer "F.Cu") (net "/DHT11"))
 (segment (start 141.01 45.06) (end 141.88 44.19) (width 0.2) (layer "F.Cu") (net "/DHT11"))
 (segment (start 121.932944 58.25) (end 106.48 58.25) (width 0.2) (layer "F.Cu") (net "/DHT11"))
 (segment (start 121.962944 58.22) (end 121.932944 58.25) (width 0.2) (layer "F.Cu") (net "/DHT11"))
 (segment (start 141.01 54.654314) (end 141.01 45.06) (width 0.2) (layer "F.Cu") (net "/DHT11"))
 (segment (start 140.61 58.324314) (end 140.61 55.054314) (width 0.2) (layer "F.Cu") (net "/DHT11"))
 (segment (start 141.01 55.22) (end 141.88 54.35) (width 0.2) (layer "F.Cu") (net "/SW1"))
 (segment (start 132.46 67.04) (end 141.01 58.49) (width 0.2) (layer "F.Cu") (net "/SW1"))
 (segment (start 141.01 58.49) (end 141.01 55.22) (width 0.2) (layer "F.Cu") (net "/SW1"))
 (segment (start 127.54 67.04) (end 132.46 67.04) (width 0.2) (layer "F.Cu") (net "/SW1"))
 (segment (start 163.25 75.5) (end 162 76.75) (width 0.2) (layer "F.Cu") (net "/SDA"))
 (segment (start 134.03 92.85) (end 136.917969 92.85) (width 0.2) (layer "F.Cu") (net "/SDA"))
 (segment (start 160.25 76.156346) (end 160.25 74.863414) (width 0.2) (layer "F.Cu") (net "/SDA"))
 (segment (start 160.843654 76.75) (end 160.25 76.156346) (width 0.2) (layer "F.Cu") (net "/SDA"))
 (segment (start 136.917969 92.85) (end 137.317969 92.45) (width 0.2) (layer "F.Cu") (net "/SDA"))
 (segment (start 158.1 47.144313) (end 158.1 41.165686) (width 0.2) (layer "F.Cu") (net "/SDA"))
 (segment (start 158.9 47.944314) (end 158.1 47.144313) (width 0.2) (layer "F.Cu") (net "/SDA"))
 (segment (start 132.88 94) (end 134.03 92.85) (width 0.2) (layer "F.Cu") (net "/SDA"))
 (segment (start 158.1 41.165686) (end 157.714314 40.78) (width 0.2) (layer "F.Cu") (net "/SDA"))
 (segment (start 146.3 92.45) (end 163.25 75.5) (width 0.2) (layer "F.Cu") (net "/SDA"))
 (segment (start 137.317969 92.45) (end 146.3 92.45) (width 0.2) (layer "F.Cu") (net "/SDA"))
 (segment (start 142.75 40.78) (end 141.88 41.65) (width 0.2) (layer "F.Cu") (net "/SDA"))
 (segment (start 158.9 73.513414) (end 158.9 47.944314) (width 0.2) (layer "F.Cu") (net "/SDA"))
 (segment (start 157.714314 40.78) (end 142.75 40.78) (width 0.2) (layer "F.Cu") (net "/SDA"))
 (segment (start 164 75.5) (end 163.25 75.5) (width 0.2) (layer "F.Cu") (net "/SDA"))
 (segment (start 162 76.75) (end 160.843654 76.75) (width 0.2) (layer "F.Cu") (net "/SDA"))
 (segment (start 160.25 74.863414) (end 158.9 73.513414) (width 0.2) (layer "F.Cu") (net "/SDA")))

